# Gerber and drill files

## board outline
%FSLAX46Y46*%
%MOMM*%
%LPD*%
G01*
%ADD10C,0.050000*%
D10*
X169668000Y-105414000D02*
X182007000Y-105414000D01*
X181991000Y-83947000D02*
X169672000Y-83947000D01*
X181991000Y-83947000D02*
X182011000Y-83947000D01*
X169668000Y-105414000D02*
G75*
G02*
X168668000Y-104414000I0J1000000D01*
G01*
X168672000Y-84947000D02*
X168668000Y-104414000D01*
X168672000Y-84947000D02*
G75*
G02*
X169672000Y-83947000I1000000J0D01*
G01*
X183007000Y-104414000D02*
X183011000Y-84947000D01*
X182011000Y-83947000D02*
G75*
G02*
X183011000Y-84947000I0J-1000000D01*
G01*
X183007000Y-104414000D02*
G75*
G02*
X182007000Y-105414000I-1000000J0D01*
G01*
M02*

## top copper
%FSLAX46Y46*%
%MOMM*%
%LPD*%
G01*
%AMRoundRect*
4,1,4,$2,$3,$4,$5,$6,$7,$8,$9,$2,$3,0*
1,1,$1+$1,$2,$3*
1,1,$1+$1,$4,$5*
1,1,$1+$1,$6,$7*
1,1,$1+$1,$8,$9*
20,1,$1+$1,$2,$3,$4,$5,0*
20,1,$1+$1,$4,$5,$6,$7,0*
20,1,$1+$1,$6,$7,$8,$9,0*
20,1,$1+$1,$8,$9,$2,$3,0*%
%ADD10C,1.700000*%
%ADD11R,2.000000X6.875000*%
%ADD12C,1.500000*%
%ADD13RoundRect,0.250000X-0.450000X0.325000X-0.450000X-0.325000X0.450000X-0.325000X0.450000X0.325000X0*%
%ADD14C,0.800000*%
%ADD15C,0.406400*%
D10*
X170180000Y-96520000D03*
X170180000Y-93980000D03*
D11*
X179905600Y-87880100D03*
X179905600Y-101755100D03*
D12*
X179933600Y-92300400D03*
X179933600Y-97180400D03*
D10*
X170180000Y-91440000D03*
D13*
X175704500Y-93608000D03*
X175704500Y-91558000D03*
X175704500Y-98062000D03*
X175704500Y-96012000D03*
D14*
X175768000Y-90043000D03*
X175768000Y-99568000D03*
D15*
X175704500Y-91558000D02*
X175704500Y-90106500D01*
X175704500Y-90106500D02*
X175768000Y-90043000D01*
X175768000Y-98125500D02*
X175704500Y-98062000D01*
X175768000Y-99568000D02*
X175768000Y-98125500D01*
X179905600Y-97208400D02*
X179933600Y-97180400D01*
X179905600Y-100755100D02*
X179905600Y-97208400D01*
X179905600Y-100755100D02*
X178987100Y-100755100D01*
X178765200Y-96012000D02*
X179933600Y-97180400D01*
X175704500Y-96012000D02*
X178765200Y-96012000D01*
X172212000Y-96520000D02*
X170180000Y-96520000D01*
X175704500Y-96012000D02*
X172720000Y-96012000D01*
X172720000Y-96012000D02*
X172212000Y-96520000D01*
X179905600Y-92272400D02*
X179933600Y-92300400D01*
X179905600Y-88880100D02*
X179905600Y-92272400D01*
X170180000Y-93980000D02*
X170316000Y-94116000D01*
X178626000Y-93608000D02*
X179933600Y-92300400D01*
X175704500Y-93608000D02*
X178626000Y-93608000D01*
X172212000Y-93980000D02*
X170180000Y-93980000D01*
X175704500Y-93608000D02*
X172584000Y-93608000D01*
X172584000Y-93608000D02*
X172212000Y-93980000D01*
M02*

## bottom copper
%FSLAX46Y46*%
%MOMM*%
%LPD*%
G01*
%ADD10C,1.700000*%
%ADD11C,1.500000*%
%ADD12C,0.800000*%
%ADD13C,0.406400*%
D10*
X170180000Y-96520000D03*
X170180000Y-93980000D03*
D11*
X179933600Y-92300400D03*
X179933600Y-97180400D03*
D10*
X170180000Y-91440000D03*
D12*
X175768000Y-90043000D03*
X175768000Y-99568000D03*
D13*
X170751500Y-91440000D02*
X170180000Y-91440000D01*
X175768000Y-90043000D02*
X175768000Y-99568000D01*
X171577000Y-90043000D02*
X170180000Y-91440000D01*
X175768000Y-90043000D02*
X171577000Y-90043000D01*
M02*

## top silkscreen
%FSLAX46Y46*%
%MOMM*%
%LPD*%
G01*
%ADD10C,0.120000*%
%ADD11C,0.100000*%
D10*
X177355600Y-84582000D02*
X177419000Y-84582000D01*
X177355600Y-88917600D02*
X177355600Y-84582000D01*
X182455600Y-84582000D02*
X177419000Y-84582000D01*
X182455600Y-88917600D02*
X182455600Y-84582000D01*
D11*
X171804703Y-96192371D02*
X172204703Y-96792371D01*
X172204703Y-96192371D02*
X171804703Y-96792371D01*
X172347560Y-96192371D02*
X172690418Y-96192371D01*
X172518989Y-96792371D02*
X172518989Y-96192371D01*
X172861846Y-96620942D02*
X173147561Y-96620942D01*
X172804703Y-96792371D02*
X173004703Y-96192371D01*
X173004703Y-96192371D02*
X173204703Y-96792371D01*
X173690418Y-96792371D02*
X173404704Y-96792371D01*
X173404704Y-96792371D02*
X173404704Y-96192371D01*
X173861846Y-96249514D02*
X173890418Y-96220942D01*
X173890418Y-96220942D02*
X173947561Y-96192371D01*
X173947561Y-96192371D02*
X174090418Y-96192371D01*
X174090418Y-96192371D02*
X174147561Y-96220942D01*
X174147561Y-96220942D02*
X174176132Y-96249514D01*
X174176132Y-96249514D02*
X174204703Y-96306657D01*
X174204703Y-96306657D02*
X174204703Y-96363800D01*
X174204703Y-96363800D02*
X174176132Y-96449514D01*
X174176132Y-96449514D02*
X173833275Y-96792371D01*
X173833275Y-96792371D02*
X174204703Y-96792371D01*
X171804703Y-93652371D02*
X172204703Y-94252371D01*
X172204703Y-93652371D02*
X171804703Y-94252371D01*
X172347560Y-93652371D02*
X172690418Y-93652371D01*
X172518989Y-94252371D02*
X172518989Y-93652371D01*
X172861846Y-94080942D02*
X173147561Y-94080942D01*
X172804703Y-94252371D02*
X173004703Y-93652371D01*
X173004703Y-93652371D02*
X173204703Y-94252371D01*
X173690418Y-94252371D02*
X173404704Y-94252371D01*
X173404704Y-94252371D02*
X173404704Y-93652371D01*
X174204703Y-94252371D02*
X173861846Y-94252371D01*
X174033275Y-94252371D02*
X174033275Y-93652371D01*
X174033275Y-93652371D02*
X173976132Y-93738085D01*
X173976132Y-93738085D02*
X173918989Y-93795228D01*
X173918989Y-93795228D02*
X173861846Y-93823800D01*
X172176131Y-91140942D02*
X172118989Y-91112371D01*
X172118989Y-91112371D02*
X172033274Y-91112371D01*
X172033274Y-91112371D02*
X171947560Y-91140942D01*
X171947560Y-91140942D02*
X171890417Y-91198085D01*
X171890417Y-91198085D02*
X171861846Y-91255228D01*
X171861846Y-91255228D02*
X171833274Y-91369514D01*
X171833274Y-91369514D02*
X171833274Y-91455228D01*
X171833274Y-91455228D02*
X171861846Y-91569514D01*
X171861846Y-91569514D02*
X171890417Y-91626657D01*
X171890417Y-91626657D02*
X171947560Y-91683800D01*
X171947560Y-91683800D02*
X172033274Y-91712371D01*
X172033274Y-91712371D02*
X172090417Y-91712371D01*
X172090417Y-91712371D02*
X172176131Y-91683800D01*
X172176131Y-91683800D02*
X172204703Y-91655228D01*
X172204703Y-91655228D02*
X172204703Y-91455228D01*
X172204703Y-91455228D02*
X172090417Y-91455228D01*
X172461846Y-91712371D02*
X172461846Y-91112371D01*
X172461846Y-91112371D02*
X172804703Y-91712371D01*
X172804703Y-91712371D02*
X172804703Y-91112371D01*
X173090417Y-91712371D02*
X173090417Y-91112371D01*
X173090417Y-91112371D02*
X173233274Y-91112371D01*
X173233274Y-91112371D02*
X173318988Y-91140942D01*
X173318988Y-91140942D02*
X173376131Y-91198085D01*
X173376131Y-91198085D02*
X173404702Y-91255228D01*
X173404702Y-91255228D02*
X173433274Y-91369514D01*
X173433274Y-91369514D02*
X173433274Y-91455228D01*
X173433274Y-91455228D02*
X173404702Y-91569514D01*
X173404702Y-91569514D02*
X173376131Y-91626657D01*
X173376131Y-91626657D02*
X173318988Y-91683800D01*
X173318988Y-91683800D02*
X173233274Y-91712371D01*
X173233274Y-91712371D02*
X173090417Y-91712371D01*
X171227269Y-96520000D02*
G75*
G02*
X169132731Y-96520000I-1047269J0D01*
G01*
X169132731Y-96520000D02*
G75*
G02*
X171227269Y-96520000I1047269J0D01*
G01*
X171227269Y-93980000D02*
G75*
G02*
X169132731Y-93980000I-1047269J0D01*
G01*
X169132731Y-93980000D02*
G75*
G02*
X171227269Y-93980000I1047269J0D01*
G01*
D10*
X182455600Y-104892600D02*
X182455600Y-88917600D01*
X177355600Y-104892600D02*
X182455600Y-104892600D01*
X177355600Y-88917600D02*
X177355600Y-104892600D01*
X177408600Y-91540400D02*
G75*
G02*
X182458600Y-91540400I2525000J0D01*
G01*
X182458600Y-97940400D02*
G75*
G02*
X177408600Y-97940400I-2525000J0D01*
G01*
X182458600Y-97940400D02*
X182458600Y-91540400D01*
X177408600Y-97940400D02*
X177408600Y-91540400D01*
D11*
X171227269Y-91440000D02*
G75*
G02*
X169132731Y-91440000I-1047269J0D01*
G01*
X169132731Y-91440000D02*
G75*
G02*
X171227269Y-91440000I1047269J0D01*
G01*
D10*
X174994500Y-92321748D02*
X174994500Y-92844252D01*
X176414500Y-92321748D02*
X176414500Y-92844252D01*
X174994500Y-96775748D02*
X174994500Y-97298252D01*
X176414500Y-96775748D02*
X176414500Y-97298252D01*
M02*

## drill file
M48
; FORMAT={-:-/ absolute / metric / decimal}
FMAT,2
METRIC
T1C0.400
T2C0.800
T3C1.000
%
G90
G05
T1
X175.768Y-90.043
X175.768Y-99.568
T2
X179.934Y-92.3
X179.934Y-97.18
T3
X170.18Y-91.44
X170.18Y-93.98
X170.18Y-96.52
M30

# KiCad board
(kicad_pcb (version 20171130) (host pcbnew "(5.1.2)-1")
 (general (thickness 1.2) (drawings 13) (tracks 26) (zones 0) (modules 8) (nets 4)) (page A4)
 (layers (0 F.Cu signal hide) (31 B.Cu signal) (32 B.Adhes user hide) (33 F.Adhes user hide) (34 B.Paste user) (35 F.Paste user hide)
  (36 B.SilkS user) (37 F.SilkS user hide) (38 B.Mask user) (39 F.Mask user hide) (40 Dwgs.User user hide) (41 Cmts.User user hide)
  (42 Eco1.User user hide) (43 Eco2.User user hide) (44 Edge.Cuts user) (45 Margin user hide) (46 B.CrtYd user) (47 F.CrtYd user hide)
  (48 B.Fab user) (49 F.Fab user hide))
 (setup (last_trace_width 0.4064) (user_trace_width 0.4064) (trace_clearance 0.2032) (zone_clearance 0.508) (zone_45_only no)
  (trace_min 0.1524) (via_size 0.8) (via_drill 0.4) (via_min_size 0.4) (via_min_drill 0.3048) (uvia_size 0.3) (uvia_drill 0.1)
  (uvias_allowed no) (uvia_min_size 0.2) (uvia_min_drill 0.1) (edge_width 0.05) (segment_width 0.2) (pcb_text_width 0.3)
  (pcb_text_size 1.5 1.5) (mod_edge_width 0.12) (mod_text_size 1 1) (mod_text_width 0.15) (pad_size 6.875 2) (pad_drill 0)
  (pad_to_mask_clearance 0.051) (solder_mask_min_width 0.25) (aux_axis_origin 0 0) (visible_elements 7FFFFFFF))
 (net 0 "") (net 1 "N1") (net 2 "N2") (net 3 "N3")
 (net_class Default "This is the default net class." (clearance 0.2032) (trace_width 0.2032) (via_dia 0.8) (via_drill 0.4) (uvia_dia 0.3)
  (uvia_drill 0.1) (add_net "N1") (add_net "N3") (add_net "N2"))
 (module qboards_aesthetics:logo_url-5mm (layer B.Cu) (at 173.736 101.854 90)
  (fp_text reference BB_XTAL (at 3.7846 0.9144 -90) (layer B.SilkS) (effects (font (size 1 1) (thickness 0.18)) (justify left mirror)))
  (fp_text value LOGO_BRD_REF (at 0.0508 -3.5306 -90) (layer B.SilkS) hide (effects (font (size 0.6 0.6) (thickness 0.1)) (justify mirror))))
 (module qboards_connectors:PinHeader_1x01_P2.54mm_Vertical (layer F.Cu) (at 170.18 96.52)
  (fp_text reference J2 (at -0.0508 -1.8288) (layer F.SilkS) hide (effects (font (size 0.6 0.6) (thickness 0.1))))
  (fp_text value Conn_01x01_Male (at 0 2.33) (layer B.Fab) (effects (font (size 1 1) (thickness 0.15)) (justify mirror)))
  (fp_circle (center 0 0) (end 0.8128 0.6604) (layer F.SilkS) (width 0.1))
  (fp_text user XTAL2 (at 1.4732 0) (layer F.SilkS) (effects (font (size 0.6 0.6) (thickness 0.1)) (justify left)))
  (pad 1 thru_hole circle (at 0 0) (size 1.7 1.7) (drill 1) (layers *.Cu *.Mask) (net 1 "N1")))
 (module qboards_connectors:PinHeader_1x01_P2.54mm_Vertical (layer F.Cu) (at 170.18 93.98)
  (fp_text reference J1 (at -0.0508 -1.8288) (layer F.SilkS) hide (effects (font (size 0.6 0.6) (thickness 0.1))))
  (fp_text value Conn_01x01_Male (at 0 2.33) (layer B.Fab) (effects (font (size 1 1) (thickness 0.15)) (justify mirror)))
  (fp_circle (center 0 0) (end 0.8128 0.6604) (layer F.SilkS) (width 0.1))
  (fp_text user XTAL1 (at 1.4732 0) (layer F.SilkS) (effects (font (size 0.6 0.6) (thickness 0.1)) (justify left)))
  (pad 1 thru_hole circle (at 0 0) (size 1.7 1.7) (drill 1) (layers *.Cu *.Mask) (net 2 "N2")))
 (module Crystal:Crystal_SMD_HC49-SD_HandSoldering (layer F.Cu) (at 179.9056 94.8176 90)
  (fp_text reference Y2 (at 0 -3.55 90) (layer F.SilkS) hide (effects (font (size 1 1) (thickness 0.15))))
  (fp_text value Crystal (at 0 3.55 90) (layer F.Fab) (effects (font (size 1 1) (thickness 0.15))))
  (fp_line (start -10.075 2.55) (end 5.9 2.55) (layer F.SilkS) (width 0.12))
  (fp_line (start -10.075 -2.55) (end -10.075 2.55) (layer F.SilkS) (width 0.12))
  (fp_line (start 5.9 -2.55) (end -10.075 -2.55) (layer F.SilkS) (width 0.12))
  (pad 2 smd rect (at 6.9375 0 90) (size 6.875 2) (layers F.Cu F.Paste F.Mask) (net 2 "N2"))
  (pad 1 smd rect (at -6.9375 0 90) (size 6.875 2) (layers F.Cu F.Paste F.Mask) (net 1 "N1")))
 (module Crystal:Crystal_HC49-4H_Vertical (layer F.Cu) (at 179.9336 97.1804 90)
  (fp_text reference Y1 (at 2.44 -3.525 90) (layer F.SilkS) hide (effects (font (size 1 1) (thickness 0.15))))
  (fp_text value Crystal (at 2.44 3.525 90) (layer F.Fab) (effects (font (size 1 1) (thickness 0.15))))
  (fp_arc (start 5.64 0) (end 5.64 -2.525) (angle 180) (layer F.SilkS) (width 0.12))
  (fp_arc (start -0.76 0) (end -0.76 -2.525) (angle -180) (layer F.SilkS) (width 0.12))
  (fp_line (start -0.76 2.525) (end 5.64 2.525) (layer F.SilkS) (width 0.12))
  (fp_line (start -0.76 -2.525) (end 5.64 -2.525) (layer F.SilkS) (width 0.12))
  (pad 2 thru_hole circle (at 4.88 0 90) (size 1.5 1.5) (drill 0.8) (layers *.Cu *.Mask) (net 2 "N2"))
  (pad 1 thru_hole circle (at 0 0 90) (size 1.5 1.5) (drill 0.8) (layers *.Cu *.Mask) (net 1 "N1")))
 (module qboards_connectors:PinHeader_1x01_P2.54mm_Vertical (layer F.Cu) (at 170.18 91.44)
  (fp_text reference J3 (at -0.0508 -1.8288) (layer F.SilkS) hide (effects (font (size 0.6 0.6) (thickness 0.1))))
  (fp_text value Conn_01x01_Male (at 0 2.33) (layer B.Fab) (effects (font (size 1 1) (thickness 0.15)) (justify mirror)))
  (fp_circle (center 0 0) (end 0.8128 0.6604) (layer F.SilkS) (width 0.1))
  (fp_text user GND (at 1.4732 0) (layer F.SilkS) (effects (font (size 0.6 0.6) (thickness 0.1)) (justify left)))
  (pad 1 thru_hole circle (at 0 0) (size 1.7 1.7) (drill 1) (layers *.Cu *.Mask) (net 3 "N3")))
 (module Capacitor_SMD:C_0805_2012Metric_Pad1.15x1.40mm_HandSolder (layer F.Cu) (at 175.7045 92.583 270)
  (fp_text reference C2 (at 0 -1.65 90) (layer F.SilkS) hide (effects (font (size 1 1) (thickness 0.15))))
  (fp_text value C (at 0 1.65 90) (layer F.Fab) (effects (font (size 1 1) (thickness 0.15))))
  (fp_line (start -0.261252 0.71) (end 0.261252 0.71) (layer F.SilkS) (width 0.12))
  (fp_line (start -0.261252 -0.71) (end 0.261252 -0.71) (layer F.SilkS) (width 0.12))
  (pad 2 smd roundrect (at 1.025 0 270) (size 1.15 1.4) (layers F.Cu F.Paste F.Mask) (roundrect_rratio 0.217391) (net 2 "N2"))
  (pad 1 smd roundrect (at -1.025 0 270) (size 1.15 1.4) (layers F.Cu F.Paste F.Mask) (roundrect_rratio 0.217391) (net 3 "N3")))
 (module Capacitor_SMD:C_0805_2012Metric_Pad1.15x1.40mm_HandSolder (layer F.Cu) (at 175.7045 97.037 270)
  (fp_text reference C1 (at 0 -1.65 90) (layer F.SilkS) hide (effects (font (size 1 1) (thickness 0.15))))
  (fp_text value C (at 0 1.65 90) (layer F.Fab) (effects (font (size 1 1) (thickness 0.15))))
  (fp_line (start -0.261252 0.71) (end 0.261252 0.71) (layer F.SilkS) (width 0.12))
  (fp_line (start -0.261252 -0.71) (end 0.261252 -0.71) (layer F.SilkS) (width 0.12))
  (pad 2 smd roundrect (at 1.025 0 270) (size 1.15 1.4) (layers F.Cu F.Paste F.Mask) (roundrect_rratio 0.217391) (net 3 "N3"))
  (pad 1 smd roundrect (at -1.025 0 270) (size 1.15 1.4) (layers F.Cu F.Paste F.Mask) (roundrect_rratio 0.217391) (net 1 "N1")))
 (gr_line (start 177.3556 84.582) (end 177.419 84.582) (layer F.SilkS) (width 0.12))
 (gr_line (start 177.3556 88.9176) (end 177.3556 84.582) (layer F.SilkS) (width 0.12))
 (gr_line (start 182.4556 84.582) (end 177.419 84.582) (layer F.SilkS) (width 0.12))
 (gr_line (start 182.4556 88.9176) (end 182.4556 84.582) (layer F.SilkS) (width 0.12))
 (gr_line (start 169.668 105.414) (end 182.007 105.414) (layer Edge.Cuts) (width 0.05))
 (gr_line (start 181.991 83.947) (end 169.672 83.947) (layer Edge.Cuts) (width 0.05))
 (gr_line (start 181.991 83.947) (end 182.011 83.947) (layer Edge.Cuts) (width 0.05))
 (gr_arc (start 169.668 104.414) (end 168.668 104.414) (angle -90) (layer Edge.Cuts) (width 0.05))
 (gr_line (start 168.672 84.947) (end 168.668 104.414) (layer Edge.Cuts) (width 0.05))
 (gr_arc (start 169.672 84.947) (end 169.672 83.947) (angle -90) (layer Edge.Cuts) (width 0.05))
 (gr_line (start 183.007 104.414) (end 183.011 84.947) (layer Edge.Cuts) (width 0.05))
 (gr_arc (start 182.011 84.947) (end 183.011 84.947) (angle -90) (layer Edge.Cuts) (width 0.05))
 (gr_arc (start 182.007 104.414) (end 182.007 105.414) (angle -90) (layer Edge.Cuts) (width 0.05))
 (segment (start 170.7515 91.44) (end 170.18 91.44) (width 0.4064) (layer B.Cu) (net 3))
 (via (at 175.768 90.043) (size 0.8) (drill 0.4) (layers F.Cu B.Cu) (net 3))
 (segment (start 175.7045 91.558) (end 175.7045 90.1065) (width 0.4064) (layer F.Cu) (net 3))
 (segment (start 175.7045 90.1065) (end 175.768 90.043) (width 0.4064) (layer F.Cu) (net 3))
 (via (at 175.768 99.568) (size 0.8) (drill 0.4) (layers F.Cu B.Cu) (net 3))
 (segment (start 175.768 90.043) (end 175.768 99.568) (width 0.4064) (layer B.Cu) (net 3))
 (segment (start 175.768 98.1255) (end 175.7045 98.062) (width 0.4064) (layer F.Cu) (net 3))
 (segment (start 175.768 99.568) (end 175.768 98.1255) (width 0.4064) (layer F.Cu) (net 3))
 (segment (start 171.577 90.043) (end 170.18 91.44) (width 0.4064) (layer B.Cu) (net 3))
 (segment (start 175.768 90.043) (end 171.577 90.043) (width 0.4064) (layer B.Cu) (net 3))
 (segment (start 179.9056 97.2084) (end 179.9336 97.1804) (width 0.4064) (layer F.Cu) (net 1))
 (segment (start 179.9056 100.7551) (end 179.9056 97.2084) (width 0.4064) (layer F.Cu) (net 1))
 (segment (start 179.9056 100.7551) (end 178.9871 100.7551) (width 0.4064) (layer F.Cu) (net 1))
 (segment (start 178.7652 96.012) (end 179.9336 97.1804) (width 0.4064) (layer F.Cu) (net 1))
 (segment (start 175.7045 96.012) (end 178.7652 96.012) (width 0.4064) (layer F.Cu) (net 1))
 (segment (start 172.212 96.52) (end 170.18 96.52) (width 0.4064) (layer F.Cu) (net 1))
 (segment (start 175.7045 96.012) (end 172.72 96.012) (width 0.4064) (layer F.Cu) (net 1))
 (segment (start 172.72 96.012) (end 172.212 96.52) (width 0.4064) (layer F.Cu) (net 1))
 (segment (start 179.9056 92.2724) (end 179.9336 92.3004) (width 0.4064) (layer F.Cu) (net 2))
 (segment (start 179.9056 88.8801) (end 179.9056 92.2724) (width 0.4064) (layer F.Cu) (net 2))
 (segment (start 170.18 93.98) (end 170.316 94.116) (width 0.4064) (layer F.Cu) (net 2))
 (segment (start 178.626 93.608) (end 179.9336 92.3004) (width 0.4064) (layer F.Cu) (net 2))
 (segment (start 175.7045 93.608) (end 178.626 93.608) (width 0.4064) (layer F.Cu) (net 2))
 (segment (start 172.212 93.98) (end 170.18 93.98) (width 0.4064) (layer F.Cu) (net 2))
 (segment (start 175.7045 93.608) (end 172.584 93.608) (width 0.4064) (layer F.Cu) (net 2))
 (segment (start 172.584 93.608) (end 172.212 93.98) (width 0.4064) (layer F.Cu) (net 2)))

